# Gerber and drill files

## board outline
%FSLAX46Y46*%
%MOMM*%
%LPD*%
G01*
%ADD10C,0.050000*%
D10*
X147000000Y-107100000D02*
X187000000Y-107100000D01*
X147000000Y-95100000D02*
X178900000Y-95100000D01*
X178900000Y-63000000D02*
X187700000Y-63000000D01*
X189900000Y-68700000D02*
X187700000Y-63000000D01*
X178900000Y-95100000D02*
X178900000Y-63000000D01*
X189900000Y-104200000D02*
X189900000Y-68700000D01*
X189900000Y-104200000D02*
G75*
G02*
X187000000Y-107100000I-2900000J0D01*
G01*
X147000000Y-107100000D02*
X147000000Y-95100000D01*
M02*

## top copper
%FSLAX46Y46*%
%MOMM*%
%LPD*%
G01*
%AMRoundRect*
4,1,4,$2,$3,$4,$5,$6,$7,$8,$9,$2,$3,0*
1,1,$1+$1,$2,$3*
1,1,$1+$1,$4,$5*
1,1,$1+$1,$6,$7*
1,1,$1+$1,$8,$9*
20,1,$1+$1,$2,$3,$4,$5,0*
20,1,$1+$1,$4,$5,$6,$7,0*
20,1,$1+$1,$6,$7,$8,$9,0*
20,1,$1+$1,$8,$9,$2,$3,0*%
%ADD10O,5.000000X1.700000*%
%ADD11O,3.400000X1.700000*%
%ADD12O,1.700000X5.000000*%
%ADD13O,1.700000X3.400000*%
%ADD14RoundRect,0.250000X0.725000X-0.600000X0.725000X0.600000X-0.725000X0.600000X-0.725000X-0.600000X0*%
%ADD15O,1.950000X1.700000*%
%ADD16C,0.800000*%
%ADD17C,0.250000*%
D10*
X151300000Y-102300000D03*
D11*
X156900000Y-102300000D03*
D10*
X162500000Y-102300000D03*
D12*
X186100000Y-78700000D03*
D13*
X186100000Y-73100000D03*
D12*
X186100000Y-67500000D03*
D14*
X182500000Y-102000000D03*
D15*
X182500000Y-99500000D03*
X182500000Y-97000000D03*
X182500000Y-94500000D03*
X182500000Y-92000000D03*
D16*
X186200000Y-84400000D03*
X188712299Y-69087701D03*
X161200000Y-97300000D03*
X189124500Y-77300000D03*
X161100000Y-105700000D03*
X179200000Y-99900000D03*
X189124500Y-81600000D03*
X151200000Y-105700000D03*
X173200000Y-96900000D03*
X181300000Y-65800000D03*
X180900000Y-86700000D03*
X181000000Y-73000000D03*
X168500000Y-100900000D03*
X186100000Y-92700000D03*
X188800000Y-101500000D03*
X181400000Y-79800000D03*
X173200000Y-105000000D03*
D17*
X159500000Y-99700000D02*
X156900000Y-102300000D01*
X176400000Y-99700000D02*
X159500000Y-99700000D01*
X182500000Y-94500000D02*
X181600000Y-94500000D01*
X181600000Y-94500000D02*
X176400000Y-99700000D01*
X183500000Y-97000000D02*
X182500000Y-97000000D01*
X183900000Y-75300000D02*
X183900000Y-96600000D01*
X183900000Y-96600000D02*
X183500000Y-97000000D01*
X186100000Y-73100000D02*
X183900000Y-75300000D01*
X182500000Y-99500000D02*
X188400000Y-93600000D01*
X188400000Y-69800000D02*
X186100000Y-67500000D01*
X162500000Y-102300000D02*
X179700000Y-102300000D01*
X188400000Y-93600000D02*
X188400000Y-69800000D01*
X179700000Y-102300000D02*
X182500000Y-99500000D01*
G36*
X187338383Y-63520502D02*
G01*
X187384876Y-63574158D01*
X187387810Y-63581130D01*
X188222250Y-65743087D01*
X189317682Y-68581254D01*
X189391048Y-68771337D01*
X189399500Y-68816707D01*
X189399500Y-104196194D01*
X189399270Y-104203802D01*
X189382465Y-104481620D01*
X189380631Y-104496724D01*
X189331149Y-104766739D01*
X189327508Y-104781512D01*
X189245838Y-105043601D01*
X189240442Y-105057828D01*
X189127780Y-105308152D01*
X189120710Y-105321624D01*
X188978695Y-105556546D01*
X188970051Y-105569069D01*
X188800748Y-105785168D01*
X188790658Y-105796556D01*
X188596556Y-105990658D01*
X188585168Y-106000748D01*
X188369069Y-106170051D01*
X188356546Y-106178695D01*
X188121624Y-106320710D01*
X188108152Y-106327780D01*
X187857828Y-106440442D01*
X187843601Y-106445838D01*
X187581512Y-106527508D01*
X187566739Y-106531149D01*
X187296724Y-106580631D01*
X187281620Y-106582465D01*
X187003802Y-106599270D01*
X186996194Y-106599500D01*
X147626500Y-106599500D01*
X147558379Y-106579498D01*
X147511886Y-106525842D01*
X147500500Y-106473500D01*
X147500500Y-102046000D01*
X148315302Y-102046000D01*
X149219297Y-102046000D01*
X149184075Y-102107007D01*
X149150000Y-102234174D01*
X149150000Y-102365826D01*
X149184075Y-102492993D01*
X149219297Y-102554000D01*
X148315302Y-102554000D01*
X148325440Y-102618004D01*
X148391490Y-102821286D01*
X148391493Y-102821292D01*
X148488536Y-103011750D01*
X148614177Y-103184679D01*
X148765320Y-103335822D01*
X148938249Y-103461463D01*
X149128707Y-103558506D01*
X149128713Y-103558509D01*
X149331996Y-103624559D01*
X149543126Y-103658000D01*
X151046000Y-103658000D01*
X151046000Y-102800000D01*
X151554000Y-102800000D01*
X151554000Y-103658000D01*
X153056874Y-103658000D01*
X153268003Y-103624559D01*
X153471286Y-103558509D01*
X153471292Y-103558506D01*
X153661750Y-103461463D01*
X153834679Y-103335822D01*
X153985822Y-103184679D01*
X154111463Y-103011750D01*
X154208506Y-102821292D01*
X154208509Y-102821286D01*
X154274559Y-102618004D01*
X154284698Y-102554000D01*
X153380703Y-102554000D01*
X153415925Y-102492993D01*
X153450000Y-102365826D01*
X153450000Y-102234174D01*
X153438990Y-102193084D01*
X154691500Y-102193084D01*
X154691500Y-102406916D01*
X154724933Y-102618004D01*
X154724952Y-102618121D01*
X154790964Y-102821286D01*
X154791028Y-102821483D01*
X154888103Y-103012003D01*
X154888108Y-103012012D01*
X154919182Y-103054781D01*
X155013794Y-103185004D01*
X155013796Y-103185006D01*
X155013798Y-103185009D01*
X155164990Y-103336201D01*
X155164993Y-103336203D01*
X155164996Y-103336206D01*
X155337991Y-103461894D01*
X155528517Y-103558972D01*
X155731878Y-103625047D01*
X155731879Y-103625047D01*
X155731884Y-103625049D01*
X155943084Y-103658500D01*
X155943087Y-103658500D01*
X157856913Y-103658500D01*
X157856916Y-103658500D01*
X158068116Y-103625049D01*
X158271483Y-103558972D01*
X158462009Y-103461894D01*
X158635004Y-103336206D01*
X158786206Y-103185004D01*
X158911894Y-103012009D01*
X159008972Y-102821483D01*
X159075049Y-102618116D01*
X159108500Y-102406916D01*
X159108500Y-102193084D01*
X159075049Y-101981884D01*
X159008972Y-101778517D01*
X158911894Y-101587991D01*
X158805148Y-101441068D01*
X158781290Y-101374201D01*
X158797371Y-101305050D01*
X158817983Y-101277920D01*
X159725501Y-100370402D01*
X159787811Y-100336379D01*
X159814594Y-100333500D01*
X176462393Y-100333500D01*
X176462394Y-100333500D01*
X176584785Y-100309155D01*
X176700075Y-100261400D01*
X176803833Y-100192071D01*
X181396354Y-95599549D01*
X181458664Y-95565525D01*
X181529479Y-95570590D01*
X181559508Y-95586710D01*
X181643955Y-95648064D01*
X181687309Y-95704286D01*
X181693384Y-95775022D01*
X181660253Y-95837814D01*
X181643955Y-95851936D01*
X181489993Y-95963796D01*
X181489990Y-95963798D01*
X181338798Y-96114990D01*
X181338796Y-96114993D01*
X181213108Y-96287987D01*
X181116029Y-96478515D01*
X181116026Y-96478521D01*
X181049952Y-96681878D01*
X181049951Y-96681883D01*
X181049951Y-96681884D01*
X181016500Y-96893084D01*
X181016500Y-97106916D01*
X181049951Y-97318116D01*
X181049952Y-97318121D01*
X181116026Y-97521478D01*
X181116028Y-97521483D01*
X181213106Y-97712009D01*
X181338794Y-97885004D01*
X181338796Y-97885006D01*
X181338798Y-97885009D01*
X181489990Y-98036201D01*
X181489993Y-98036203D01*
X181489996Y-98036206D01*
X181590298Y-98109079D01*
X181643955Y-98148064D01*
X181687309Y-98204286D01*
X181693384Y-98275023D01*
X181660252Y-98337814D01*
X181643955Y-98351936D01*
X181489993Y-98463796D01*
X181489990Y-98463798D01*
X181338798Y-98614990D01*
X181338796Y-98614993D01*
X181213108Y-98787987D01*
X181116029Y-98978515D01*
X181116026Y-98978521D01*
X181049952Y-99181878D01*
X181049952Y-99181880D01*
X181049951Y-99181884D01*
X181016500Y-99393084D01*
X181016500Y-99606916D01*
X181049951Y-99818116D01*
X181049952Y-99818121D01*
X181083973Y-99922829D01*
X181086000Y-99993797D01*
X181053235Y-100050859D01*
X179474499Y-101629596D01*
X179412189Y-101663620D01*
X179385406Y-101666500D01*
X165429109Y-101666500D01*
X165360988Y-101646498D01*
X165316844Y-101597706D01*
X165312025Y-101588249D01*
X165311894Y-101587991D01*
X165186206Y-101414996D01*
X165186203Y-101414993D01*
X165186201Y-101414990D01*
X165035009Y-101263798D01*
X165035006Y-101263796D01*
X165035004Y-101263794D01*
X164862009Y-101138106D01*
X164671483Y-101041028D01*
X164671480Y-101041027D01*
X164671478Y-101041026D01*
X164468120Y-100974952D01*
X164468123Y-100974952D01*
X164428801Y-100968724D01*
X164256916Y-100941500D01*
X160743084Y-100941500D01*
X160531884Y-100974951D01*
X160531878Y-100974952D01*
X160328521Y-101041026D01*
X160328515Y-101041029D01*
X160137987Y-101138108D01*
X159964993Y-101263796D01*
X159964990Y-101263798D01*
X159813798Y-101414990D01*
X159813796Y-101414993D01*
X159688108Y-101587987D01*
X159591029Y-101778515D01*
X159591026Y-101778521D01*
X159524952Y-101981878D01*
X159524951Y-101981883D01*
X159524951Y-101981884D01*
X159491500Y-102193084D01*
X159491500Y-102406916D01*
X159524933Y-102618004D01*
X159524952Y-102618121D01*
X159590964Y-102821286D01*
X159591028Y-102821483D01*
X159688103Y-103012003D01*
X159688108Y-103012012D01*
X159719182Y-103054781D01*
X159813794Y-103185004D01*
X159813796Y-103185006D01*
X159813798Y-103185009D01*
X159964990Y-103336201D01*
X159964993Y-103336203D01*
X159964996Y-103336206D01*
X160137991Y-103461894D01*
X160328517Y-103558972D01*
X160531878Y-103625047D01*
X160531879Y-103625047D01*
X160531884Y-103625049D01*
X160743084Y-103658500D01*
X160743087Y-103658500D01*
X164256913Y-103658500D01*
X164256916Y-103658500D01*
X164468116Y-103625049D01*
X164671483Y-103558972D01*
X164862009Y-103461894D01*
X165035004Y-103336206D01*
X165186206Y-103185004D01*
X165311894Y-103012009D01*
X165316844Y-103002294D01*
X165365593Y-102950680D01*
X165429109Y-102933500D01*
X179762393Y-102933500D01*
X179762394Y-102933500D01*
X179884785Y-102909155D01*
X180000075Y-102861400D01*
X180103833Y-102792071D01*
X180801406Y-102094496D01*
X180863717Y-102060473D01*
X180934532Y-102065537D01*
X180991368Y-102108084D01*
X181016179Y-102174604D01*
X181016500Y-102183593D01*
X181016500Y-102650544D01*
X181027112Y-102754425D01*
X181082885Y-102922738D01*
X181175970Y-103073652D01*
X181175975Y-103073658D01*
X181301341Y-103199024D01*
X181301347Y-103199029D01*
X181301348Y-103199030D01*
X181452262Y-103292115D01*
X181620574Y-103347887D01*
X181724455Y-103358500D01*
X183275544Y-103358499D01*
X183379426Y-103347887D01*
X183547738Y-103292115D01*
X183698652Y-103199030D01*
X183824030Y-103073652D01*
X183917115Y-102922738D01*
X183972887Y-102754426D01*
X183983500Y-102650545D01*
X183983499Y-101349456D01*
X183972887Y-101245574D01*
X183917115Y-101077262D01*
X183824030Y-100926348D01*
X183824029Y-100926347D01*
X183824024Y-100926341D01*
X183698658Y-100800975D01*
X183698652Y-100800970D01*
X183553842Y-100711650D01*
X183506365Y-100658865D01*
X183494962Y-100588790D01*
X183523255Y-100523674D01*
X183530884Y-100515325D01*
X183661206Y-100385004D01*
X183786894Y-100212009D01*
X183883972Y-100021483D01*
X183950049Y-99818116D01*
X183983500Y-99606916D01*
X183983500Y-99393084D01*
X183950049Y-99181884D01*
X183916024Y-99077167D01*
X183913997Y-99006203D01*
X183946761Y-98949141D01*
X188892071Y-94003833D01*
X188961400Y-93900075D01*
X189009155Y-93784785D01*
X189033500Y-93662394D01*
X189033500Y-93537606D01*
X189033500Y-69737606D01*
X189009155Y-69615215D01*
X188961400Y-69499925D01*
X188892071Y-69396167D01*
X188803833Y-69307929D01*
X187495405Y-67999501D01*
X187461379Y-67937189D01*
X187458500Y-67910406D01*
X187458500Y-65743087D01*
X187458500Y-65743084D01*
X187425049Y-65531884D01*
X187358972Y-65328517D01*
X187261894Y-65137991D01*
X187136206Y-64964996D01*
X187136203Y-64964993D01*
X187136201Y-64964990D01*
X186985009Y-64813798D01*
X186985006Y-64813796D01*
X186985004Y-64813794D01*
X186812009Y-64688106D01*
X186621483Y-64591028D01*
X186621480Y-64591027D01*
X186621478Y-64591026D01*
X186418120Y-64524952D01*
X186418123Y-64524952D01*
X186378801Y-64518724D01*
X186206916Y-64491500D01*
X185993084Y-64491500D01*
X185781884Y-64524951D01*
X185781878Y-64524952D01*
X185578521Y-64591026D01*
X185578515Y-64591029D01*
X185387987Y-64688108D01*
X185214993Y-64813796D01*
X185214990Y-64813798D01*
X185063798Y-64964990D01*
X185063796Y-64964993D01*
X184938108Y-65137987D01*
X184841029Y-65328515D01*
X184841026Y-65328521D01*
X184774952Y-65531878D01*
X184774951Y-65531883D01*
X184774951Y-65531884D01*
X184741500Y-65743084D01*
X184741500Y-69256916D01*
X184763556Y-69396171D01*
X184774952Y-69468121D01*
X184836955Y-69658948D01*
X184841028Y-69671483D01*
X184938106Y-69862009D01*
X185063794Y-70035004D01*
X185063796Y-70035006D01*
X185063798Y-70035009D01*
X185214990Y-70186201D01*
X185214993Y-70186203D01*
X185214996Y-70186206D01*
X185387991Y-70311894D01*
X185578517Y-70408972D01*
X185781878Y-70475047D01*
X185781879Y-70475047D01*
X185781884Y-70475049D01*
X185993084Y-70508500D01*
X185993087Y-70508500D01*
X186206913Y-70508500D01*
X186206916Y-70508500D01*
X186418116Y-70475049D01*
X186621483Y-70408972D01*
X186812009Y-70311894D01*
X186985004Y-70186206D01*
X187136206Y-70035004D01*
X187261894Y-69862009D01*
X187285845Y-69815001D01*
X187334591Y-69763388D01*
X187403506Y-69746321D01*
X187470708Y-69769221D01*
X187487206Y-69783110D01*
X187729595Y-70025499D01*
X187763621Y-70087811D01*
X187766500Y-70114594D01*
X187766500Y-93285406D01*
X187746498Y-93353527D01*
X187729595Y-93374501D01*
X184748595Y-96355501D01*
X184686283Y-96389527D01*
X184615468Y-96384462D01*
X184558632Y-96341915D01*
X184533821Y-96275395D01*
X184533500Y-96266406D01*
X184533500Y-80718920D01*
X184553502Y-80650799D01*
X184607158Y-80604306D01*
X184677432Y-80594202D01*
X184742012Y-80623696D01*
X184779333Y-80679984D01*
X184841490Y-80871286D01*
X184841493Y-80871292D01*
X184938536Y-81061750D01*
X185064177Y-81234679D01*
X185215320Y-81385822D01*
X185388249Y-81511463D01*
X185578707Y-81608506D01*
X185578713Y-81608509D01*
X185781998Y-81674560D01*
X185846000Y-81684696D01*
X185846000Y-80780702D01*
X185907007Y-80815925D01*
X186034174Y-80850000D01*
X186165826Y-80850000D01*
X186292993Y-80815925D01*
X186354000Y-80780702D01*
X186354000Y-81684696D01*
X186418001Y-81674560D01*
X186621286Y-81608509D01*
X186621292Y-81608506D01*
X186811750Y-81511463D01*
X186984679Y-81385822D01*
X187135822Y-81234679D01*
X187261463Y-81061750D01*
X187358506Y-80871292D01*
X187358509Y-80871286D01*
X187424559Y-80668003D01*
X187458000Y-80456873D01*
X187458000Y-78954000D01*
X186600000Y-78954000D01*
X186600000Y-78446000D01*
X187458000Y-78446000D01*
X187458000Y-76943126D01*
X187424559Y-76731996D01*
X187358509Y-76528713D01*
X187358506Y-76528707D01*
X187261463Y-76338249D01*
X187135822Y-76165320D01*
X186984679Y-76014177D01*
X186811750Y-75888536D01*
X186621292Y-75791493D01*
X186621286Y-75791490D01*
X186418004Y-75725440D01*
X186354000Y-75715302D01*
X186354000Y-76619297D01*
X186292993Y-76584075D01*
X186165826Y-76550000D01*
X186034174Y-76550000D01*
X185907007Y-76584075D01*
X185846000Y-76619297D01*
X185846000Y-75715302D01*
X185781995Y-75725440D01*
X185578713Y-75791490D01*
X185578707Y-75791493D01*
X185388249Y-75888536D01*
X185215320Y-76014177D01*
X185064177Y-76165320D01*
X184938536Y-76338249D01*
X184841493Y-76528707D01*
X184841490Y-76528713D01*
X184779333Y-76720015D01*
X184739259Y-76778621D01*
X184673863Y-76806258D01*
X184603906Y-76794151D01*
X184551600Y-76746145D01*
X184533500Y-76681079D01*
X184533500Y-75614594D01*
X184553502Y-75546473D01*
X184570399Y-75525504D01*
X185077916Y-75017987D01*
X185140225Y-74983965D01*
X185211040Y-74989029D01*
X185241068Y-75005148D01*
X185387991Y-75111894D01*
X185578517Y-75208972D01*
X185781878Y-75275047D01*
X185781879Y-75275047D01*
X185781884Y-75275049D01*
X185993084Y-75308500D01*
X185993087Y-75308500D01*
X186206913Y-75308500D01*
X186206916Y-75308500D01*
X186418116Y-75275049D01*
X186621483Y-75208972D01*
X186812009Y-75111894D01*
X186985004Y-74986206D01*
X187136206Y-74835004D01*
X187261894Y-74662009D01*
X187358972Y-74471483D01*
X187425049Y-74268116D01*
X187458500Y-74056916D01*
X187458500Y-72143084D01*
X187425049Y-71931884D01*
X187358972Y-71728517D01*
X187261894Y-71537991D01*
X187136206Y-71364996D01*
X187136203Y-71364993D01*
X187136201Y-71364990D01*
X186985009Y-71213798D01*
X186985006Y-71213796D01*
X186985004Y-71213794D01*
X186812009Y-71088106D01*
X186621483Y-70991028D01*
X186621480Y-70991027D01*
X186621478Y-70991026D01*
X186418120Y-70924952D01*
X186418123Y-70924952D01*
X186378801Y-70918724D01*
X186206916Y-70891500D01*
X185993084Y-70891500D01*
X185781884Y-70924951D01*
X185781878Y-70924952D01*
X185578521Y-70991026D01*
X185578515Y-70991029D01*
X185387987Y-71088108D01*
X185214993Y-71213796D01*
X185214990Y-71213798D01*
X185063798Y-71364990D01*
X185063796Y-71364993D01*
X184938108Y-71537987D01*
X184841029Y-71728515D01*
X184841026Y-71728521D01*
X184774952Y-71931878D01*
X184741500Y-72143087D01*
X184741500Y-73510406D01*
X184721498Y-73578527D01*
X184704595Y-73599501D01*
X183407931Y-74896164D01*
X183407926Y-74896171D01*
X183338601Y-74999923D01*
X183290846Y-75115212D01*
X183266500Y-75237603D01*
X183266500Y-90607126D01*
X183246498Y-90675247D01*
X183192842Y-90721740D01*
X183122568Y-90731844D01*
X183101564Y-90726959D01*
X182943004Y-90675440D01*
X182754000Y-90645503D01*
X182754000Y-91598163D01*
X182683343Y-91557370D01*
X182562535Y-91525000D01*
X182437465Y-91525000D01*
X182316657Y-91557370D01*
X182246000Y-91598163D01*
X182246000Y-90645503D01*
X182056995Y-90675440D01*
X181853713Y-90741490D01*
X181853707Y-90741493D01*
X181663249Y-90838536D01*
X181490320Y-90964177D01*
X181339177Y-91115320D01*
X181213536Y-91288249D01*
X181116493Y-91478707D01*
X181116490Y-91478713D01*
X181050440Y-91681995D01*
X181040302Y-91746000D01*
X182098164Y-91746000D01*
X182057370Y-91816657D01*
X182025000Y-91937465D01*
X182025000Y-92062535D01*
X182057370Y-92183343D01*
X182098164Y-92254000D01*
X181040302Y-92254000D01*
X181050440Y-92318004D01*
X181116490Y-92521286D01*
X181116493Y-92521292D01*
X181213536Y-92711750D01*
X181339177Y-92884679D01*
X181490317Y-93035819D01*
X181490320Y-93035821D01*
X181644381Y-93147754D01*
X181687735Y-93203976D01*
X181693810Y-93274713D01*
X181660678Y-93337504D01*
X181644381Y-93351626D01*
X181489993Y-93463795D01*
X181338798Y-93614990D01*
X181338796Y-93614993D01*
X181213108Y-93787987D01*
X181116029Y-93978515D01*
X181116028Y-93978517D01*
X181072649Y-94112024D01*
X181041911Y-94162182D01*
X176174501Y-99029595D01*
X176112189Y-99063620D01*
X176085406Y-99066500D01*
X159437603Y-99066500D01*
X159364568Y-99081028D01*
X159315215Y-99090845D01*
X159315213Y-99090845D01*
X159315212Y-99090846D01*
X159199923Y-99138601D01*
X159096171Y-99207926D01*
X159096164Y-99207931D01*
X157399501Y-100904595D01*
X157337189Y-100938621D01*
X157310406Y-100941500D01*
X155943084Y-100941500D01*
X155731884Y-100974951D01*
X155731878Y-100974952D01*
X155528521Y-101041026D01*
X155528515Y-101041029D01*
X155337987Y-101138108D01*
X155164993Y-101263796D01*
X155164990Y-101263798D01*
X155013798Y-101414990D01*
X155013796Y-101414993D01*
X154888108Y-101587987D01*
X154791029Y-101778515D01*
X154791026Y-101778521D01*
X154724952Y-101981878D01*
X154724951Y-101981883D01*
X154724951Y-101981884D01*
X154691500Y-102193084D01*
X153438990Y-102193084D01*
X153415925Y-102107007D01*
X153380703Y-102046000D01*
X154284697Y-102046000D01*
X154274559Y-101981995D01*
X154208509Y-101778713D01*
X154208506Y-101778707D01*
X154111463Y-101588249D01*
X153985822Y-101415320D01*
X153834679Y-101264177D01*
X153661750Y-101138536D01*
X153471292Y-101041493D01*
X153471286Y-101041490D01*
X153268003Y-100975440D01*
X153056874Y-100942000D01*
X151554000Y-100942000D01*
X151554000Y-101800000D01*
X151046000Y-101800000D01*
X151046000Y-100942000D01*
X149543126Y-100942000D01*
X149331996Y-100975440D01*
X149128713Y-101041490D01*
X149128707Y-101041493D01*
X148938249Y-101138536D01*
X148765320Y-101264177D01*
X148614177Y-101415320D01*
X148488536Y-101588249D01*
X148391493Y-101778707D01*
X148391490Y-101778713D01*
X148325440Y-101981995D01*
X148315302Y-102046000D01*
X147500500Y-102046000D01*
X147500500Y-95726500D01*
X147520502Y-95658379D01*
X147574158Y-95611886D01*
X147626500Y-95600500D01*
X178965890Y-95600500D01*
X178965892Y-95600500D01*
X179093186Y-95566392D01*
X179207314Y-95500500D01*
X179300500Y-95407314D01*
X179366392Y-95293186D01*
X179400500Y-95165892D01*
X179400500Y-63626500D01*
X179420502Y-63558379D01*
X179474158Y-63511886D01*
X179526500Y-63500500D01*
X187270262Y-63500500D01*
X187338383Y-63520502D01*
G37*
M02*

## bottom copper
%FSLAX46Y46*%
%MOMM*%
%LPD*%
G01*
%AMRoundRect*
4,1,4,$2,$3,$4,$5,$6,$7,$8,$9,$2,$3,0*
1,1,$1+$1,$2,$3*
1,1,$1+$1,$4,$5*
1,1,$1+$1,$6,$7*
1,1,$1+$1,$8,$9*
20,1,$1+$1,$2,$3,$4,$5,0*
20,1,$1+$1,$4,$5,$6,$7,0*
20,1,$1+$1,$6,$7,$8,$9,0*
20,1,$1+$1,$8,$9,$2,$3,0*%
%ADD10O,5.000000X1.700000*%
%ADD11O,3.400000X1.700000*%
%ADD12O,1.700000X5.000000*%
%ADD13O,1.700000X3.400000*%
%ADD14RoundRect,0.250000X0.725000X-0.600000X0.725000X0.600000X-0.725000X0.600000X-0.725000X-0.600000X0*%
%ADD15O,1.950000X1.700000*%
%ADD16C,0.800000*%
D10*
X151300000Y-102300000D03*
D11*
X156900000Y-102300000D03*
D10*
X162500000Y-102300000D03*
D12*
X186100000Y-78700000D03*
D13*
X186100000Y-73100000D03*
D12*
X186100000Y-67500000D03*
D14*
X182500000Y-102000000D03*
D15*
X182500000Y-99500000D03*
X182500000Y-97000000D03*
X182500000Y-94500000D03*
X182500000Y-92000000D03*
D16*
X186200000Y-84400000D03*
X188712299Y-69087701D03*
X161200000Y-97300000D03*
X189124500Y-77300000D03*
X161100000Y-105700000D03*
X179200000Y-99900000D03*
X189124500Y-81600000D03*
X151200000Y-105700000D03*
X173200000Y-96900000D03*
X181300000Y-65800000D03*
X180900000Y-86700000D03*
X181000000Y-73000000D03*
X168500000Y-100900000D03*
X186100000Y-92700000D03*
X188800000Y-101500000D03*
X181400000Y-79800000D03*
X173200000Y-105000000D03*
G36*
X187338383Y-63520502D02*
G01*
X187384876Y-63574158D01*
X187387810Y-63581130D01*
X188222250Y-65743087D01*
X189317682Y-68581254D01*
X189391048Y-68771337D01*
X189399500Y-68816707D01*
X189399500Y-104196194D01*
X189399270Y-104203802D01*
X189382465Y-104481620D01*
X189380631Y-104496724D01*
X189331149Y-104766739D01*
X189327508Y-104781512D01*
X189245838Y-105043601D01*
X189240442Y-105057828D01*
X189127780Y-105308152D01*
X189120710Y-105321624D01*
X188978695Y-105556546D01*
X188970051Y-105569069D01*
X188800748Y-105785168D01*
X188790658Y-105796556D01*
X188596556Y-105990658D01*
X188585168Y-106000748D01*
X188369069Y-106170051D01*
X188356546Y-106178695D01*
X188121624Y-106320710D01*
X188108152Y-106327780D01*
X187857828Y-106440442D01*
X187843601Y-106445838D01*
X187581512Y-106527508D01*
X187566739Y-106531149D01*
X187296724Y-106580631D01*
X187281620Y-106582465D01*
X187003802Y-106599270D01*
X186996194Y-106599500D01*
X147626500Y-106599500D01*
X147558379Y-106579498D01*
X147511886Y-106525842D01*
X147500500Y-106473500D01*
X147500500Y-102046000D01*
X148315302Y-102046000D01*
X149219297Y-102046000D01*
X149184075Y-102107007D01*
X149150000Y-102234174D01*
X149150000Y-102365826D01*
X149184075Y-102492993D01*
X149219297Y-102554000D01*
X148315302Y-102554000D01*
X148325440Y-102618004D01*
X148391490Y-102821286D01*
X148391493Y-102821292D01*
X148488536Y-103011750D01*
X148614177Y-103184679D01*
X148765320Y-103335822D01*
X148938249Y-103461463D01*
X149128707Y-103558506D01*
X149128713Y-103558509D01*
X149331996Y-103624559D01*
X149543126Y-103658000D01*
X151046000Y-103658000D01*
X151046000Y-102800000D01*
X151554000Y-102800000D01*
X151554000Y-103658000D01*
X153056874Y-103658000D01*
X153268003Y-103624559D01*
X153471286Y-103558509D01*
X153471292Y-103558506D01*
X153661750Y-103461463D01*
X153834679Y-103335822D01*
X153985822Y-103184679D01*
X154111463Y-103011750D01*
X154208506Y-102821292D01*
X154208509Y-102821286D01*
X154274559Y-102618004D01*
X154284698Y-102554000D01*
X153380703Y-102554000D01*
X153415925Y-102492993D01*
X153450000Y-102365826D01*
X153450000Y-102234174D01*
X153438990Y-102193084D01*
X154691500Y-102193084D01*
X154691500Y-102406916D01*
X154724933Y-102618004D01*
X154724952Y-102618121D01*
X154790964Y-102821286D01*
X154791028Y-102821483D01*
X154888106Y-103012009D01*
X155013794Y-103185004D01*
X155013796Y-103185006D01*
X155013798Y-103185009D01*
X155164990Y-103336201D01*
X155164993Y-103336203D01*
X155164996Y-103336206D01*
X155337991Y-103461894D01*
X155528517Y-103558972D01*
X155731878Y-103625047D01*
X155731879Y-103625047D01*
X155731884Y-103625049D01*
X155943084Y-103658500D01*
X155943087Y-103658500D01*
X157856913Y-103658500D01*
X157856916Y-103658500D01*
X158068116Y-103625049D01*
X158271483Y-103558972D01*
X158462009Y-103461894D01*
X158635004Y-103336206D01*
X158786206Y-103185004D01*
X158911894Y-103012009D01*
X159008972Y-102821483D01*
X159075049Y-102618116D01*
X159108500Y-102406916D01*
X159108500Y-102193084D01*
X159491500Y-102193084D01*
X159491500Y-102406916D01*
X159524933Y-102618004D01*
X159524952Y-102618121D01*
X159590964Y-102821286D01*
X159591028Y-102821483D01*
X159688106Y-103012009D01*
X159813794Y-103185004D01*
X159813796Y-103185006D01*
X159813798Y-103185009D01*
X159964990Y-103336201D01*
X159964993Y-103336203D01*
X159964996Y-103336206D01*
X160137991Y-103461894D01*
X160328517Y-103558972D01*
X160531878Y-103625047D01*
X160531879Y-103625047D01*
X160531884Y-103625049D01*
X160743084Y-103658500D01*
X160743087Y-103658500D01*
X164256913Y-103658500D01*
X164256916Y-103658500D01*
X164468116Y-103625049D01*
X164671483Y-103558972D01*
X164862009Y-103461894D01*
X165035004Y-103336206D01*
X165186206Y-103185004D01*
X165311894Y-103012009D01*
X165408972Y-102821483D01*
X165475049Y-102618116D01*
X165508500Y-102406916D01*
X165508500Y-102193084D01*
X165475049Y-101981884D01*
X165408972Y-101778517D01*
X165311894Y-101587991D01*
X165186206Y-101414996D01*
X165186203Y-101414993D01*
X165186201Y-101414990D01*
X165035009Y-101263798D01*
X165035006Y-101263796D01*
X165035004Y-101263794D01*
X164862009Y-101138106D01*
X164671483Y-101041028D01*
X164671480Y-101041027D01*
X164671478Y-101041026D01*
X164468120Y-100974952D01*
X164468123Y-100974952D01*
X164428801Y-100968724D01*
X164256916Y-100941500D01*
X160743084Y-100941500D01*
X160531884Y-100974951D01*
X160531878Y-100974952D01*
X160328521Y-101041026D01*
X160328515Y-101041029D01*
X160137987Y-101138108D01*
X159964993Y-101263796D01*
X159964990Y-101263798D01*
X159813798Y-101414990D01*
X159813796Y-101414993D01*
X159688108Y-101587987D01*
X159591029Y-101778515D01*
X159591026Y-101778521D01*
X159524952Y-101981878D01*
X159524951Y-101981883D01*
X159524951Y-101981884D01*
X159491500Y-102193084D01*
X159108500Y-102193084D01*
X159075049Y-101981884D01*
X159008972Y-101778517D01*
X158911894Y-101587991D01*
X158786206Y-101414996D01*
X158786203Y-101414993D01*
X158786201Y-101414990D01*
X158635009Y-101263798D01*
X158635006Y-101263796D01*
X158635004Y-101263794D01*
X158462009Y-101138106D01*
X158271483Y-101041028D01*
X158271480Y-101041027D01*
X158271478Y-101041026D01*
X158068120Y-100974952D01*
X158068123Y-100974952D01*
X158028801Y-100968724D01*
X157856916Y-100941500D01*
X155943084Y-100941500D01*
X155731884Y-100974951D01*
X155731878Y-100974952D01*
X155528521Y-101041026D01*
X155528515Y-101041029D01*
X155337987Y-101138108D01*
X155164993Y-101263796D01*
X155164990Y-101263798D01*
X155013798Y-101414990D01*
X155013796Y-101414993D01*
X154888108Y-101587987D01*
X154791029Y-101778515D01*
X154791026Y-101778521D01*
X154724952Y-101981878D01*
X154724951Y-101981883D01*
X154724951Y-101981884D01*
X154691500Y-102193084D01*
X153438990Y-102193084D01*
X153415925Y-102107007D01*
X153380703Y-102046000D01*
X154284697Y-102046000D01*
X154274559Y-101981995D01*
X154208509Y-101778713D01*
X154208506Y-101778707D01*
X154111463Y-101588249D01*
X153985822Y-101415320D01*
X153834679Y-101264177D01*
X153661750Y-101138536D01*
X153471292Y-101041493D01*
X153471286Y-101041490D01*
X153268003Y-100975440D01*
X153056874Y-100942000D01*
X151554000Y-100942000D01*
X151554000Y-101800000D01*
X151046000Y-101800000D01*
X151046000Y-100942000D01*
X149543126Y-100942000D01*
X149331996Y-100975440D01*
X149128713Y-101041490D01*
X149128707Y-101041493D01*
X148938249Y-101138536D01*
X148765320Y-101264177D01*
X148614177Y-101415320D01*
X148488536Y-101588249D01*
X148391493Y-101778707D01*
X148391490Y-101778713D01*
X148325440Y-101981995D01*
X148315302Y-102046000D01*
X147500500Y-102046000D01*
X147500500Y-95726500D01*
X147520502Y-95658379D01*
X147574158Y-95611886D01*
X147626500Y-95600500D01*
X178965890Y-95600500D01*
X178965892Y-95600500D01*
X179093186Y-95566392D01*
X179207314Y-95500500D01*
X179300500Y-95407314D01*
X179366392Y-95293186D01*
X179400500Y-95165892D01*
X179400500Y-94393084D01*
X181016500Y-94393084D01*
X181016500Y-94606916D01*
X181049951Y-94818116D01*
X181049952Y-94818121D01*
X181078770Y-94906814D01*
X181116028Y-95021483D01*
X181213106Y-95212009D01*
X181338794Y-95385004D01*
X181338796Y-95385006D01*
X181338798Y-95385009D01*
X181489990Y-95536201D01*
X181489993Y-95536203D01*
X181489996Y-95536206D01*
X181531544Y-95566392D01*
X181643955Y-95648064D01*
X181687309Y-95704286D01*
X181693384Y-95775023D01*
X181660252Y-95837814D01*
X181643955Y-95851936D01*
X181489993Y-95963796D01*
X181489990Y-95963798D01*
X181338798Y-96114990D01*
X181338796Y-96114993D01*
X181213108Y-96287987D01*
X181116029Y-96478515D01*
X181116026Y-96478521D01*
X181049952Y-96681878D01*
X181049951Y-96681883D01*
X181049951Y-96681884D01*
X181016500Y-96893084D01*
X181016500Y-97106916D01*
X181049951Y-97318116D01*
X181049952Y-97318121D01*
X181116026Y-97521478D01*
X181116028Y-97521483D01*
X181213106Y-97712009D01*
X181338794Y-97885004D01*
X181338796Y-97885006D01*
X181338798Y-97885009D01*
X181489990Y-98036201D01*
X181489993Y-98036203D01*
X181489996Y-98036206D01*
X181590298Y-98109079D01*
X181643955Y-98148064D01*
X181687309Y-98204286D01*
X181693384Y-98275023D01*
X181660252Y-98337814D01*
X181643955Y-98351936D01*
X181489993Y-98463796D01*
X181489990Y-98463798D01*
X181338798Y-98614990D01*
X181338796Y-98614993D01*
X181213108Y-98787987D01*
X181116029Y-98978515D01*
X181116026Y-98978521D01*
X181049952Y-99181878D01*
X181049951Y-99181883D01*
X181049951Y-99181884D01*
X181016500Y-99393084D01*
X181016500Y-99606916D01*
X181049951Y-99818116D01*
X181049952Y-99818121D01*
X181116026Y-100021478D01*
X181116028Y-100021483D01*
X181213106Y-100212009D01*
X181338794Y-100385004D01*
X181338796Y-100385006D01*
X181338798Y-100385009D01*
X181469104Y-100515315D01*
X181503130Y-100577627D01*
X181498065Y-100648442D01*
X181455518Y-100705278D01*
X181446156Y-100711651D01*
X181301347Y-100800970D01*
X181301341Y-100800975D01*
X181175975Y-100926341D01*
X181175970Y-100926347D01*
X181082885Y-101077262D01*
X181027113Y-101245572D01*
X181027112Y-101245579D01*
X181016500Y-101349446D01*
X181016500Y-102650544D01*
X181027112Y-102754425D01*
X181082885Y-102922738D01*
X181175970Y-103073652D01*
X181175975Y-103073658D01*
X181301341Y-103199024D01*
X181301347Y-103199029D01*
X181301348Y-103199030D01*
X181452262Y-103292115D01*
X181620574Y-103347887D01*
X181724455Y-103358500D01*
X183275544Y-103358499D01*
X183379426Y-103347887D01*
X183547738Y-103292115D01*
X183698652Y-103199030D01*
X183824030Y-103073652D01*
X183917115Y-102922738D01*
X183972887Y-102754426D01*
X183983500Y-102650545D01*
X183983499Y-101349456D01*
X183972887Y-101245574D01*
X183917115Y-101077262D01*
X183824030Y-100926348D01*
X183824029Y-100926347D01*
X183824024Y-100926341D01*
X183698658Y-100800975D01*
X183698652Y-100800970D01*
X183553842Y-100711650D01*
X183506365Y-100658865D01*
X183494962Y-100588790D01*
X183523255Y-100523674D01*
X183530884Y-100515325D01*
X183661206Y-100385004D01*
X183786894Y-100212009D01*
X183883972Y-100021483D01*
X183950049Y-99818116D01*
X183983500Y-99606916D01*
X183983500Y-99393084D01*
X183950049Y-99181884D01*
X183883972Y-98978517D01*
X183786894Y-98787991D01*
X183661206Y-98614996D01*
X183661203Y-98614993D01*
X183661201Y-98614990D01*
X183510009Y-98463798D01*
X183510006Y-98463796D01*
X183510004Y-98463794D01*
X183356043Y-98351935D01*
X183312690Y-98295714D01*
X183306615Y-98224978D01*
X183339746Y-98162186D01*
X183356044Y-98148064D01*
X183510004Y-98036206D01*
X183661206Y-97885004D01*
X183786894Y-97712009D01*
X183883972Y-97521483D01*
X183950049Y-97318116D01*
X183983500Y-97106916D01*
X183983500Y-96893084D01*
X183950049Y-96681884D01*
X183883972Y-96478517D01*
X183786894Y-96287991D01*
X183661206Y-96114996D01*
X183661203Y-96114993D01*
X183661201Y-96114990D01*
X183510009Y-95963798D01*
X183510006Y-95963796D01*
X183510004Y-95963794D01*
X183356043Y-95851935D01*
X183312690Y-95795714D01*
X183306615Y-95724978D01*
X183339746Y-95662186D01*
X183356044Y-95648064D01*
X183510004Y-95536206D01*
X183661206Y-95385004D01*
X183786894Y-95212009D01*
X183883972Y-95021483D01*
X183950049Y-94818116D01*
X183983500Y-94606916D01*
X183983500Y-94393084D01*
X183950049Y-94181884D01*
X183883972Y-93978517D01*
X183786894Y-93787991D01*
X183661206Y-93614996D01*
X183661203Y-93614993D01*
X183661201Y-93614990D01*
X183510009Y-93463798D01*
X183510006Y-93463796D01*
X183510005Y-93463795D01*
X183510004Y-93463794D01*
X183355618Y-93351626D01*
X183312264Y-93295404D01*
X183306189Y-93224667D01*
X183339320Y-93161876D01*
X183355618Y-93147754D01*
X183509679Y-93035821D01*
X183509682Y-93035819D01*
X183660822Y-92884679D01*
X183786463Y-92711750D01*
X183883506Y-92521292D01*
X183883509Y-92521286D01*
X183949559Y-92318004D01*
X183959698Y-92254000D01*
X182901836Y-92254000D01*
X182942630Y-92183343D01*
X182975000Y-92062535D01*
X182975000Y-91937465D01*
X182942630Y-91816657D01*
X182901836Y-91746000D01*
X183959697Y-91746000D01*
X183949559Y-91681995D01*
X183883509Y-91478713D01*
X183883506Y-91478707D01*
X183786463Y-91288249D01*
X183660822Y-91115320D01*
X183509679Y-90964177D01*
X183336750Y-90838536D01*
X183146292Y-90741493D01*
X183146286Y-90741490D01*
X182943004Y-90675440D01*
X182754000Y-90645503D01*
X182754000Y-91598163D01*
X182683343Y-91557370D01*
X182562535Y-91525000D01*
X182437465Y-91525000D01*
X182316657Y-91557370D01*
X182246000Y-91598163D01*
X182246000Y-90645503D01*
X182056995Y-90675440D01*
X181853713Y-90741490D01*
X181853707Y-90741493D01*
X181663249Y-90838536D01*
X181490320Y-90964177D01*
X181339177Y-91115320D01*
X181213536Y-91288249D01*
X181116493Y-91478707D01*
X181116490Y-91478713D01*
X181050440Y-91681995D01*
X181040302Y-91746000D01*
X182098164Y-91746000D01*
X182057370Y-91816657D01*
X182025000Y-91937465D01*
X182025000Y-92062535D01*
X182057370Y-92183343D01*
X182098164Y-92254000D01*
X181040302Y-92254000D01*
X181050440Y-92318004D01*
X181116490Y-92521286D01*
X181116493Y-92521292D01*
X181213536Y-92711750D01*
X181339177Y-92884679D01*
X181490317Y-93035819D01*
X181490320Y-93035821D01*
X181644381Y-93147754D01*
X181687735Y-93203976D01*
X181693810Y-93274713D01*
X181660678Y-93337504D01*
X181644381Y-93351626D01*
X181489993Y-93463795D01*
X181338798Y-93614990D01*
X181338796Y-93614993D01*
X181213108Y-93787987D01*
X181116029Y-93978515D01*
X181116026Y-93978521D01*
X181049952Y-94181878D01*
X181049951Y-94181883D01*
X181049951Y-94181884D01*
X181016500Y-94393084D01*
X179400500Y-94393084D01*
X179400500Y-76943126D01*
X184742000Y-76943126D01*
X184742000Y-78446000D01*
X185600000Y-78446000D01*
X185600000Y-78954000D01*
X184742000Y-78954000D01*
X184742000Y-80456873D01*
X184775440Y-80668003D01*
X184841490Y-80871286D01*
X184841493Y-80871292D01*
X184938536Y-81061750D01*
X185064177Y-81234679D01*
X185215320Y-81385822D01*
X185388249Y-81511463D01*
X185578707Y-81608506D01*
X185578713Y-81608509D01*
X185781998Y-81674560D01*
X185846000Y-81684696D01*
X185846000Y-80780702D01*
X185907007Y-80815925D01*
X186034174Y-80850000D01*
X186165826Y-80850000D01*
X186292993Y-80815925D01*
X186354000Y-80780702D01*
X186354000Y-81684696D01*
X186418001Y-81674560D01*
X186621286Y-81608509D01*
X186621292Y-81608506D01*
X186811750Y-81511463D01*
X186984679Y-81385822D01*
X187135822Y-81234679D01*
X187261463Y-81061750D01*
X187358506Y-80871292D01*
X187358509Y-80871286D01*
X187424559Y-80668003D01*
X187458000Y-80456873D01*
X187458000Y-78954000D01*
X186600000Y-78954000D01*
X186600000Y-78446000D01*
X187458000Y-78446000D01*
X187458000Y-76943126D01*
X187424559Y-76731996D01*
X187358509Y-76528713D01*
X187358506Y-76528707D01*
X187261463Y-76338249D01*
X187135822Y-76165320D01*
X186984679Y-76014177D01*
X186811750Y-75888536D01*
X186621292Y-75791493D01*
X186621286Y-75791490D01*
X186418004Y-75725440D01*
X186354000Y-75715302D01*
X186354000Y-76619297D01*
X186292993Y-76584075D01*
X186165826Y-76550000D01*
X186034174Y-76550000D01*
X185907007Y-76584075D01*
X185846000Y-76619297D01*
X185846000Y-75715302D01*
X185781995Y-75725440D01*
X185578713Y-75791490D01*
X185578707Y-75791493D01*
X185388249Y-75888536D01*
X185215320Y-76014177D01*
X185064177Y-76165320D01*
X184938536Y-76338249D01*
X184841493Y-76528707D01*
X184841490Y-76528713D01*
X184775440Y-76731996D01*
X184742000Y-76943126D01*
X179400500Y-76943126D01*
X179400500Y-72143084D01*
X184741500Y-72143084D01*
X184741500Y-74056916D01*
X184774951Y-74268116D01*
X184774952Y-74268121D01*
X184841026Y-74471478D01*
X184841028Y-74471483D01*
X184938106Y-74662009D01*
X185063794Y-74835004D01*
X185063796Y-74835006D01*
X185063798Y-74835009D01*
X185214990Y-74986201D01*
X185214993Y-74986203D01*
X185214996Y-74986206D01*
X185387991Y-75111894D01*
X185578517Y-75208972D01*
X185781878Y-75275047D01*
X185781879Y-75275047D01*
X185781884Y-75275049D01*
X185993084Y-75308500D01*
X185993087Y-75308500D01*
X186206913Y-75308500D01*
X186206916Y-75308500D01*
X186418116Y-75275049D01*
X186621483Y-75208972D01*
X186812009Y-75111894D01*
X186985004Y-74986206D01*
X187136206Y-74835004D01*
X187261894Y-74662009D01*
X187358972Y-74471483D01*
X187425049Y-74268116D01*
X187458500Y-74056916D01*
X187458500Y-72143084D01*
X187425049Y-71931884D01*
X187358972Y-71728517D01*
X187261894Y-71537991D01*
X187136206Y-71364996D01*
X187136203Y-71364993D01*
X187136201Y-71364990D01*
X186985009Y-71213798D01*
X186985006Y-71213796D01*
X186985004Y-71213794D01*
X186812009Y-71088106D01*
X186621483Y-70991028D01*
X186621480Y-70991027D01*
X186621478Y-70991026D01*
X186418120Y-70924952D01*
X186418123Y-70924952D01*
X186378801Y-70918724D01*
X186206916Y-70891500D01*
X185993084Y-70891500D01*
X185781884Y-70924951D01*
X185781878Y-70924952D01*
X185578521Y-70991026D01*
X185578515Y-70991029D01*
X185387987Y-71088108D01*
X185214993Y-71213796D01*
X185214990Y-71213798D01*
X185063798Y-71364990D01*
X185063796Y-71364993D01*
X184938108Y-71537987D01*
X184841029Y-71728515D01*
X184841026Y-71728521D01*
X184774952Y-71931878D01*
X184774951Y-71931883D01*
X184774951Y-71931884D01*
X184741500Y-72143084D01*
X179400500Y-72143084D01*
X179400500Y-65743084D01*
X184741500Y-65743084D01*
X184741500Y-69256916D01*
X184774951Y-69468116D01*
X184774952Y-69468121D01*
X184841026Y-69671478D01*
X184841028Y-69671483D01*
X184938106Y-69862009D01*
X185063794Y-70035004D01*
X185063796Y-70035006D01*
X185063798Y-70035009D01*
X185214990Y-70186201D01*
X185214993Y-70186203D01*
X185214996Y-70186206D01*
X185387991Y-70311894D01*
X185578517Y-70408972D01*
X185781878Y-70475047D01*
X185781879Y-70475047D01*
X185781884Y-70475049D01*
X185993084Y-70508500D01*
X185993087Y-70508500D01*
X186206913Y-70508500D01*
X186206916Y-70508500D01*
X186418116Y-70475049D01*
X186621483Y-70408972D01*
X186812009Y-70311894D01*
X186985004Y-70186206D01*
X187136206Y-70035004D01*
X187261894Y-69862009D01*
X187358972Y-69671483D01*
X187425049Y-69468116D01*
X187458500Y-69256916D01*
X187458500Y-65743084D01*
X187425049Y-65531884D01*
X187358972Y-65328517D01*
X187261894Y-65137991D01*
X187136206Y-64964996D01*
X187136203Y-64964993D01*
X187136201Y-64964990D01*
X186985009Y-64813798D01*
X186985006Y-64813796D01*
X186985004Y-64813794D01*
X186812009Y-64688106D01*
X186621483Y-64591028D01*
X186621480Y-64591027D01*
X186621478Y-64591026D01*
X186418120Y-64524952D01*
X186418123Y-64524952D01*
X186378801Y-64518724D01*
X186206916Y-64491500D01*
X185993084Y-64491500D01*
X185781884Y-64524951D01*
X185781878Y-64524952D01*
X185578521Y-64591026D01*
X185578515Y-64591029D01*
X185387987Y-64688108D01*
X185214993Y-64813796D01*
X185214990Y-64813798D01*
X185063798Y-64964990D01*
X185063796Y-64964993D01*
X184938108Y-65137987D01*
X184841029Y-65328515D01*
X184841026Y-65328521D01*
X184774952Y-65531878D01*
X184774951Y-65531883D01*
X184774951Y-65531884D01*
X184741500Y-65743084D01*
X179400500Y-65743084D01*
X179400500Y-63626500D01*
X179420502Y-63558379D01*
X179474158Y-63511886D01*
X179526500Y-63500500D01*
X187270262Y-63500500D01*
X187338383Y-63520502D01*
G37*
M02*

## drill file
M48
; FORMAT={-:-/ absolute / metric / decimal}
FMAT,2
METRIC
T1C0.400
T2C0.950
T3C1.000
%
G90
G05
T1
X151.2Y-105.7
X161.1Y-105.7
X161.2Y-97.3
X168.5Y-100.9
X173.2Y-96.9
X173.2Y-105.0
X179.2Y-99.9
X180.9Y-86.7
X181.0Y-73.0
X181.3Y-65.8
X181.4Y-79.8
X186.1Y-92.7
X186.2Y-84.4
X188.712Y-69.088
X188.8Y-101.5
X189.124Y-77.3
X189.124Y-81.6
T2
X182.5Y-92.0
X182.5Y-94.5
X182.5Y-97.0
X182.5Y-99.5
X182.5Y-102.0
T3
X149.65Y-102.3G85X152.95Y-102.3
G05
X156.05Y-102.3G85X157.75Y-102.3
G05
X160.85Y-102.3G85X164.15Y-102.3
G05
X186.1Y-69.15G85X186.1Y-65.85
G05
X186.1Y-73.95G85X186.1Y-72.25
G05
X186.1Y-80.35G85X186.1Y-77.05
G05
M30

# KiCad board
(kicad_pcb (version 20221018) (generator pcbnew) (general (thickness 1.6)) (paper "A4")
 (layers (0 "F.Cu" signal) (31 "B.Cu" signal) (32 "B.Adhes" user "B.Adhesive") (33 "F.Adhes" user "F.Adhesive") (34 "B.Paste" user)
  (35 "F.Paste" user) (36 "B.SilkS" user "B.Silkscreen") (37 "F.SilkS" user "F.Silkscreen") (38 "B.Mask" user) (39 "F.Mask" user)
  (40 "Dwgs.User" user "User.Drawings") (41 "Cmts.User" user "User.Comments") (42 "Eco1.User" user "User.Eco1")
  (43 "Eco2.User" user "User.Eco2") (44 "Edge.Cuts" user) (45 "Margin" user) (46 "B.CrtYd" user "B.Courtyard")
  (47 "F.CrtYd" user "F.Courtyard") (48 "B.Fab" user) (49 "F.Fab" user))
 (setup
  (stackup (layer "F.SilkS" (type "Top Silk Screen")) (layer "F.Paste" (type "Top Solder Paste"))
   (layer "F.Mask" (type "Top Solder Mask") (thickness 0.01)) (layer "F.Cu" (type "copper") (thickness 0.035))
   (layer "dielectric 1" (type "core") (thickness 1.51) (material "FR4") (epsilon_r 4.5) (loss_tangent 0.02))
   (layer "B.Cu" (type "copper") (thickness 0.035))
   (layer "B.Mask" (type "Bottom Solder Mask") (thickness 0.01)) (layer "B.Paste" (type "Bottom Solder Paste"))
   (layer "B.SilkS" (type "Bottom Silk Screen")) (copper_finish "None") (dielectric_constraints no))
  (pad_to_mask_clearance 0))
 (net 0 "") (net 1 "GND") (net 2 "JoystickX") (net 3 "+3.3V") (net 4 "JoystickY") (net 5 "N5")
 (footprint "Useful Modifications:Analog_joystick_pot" (layer "F.Cu") (at 156.9 102.3 90)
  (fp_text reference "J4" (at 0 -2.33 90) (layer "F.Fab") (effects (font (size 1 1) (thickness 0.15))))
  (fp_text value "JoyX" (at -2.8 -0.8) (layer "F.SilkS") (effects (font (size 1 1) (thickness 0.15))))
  (pad "1" thru_hole oval (at 0 -5.6 90) (size 1.7 5) (drill oval 1 4.3) (layers "*.Cu" "*.Mask") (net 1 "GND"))
  (pad "2" thru_hole oval (at 0 0 90) (size 1.7 3.4) (drill oval 1 2.7) (layers "*.Cu" "*.Mask") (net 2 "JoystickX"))
  (pad "3" thru_hole oval (at 0 5.6 90) (size 1.7 5) (drill oval 1 4.3) (layers "*.Cu" "*.Mask") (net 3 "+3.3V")))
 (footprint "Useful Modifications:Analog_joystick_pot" (layer "F.Cu") (at 186.1 73.1 180)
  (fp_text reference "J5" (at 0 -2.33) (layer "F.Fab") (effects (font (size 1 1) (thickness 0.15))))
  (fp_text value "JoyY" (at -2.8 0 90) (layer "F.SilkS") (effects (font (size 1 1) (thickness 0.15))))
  (pad "1" thru_hole oval (at 0 -5.6 180) (size 1.7 5) (drill oval 1 4.3) (layers "*.Cu" "*.Mask") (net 1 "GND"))
  (pad "2" thru_hole oval (at 0 0 180) (size 1.7 3.4) (drill oval 1 2.7) (layers "*.Cu" "*.Mask") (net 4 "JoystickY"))
  (pad "3" thru_hole oval (at 0 5.6 180) (size 1.7 5) (drill oval 1 4.3) (layers "*.Cu" "*.Mask") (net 3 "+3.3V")))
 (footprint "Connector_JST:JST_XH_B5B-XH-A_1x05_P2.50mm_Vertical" (layer "F.Cu") (at 182.5 102 90)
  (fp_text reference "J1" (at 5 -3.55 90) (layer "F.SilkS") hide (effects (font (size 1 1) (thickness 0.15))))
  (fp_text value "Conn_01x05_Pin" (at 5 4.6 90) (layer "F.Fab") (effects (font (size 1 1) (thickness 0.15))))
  (pad "1" thru_hole roundrect (at 0 0 90) (size 1.7 1.95) (drill 0.95) (layers "*.Cu" "*.Mask") (roundrect_rratio 0.147059) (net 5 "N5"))
  (pad "2" thru_hole oval (at 2.5 0 90) (size 1.7 1.95) (drill 0.95) (layers "*.Cu" "*.Mask") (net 3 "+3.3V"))
  (pad "3" thru_hole oval (at 5 0 90) (size 1.7 1.95) (drill 0.95) (layers "*.Cu" "*.Mask") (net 4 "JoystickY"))
  (pad "4" thru_hole oval (at 7.5 0 90) (size 1.7 1.95) (drill 0.95) (layers "*.Cu" "*.Mask") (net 2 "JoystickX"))
  (pad "5" thru_hole oval (at 10 0 90) (size 1.7 1.95) (drill 0.95) (layers "*.Cu" "*.Mask") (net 1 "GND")))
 (gr_line (start 147 107.1) (end 187 107.1) (stroke (width 0.05) (type default)) (layer "Edge.Cuts"))
 (gr_line (start 147 95.1) (end 178.9 95.1) (stroke (width 0.05) (type default)) (layer "Edge.Cuts"))
 (gr_line (start 178.9 63) (end 187.7 63) (stroke (width 0.05) (type default)) (layer "Edge.Cuts"))
 (gr_line (start 189.9 68.7) (end 187.7 63) (stroke (width 0.05) (type default)) (layer "Edge.Cuts"))
 (gr_line (start 178.9 95.1) (end 178.9 63) (stroke (width 0.05) (type default)) (layer "Edge.Cuts"))
 (gr_line (start 189.9 104.2) (end 189.9 68.7) (stroke (width 0.05) (type default)) (layer "Edge.Cuts"))
 (gr_arc (start 189.9 104.2) (mid 189.05061 106.25061) (end 187 107.1) (stroke (width 0.05) (type default)) (layer "Edge.Cuts"))
 (gr_line (start 147 107.1) (end 147 95.1) (stroke (width 0.05) (type default)) (layer "Edge.Cuts"))
 (via (at 186.2 84.4) (size 0.8) (drill 0.4) (layers "F.Cu" "B.Cu") (free) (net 1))
 (via (at 188.712299 69.087701) (size 0.8) (drill 0.4) (layers "F.Cu" "B.Cu") (free) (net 1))
 (via (at 161.2 97.3) (size 0.8) (drill 0.4) (layers "F.Cu" "B.Cu") (free) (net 1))
 (via (at 189.1245 77.3) (size 0.8) (drill 0.4) (layers "F.Cu" "B.Cu") (free) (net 1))
 (via (at 161.1 105.7) (size 0.8) (drill 0.4) (layers "F.Cu" "B.Cu") (free) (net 1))
 (via (at 179.2 99.9) (size 0.8) (drill 0.4) (layers "F.Cu" "B.Cu") (free) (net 1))
 (via (at 189.1245 81.6) (size 0.8) (drill 0.4) (layers "F.Cu" "B.Cu") (free) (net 1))
 (via (at 151.2 105.7) (size 0.8) (drill 0.4) (layers "F.Cu" "B.Cu") (free) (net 1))
 (via (at 173.2 96.9) (size 0.8) (drill 0.4) (layers "F.Cu" "B.Cu") (free) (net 1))
 (via (at 181.3 65.8) (size 0.8) (drill 0.4) (layers "F.Cu" "B.Cu") (free) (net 1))
 (via (at 180.9 86.7) (size 0.8) (drill 0.4) (layers "F.Cu" "B.Cu") (free) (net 1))
 (via (at 181 73) (size 0.8) (drill 0.4) (layers "F.Cu" "B.Cu") (free) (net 1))
 (via (at 168.5 100.9) (size 0.8) (drill 0.4) (layers "F.Cu" "B.Cu") (free) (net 1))
 (via (at 186.1 92.7) (size 0.8) (drill 0.4) (layers "F.Cu" "B.Cu") (free) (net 1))
 (via (at 188.8 101.5) (size 0.8) (drill 0.4) (layers "F.Cu" "B.Cu") (free) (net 1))
 (via (at 181.4 79.8) (size 0.8) (drill 0.4) (layers "F.Cu" "B.Cu") (free) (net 1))
 (via (at 173.2 105) (size 0.8) (drill 0.4) (layers "F.Cu" "B.Cu") (free) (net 1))
 (segment (start 159.5 99.7) (end 156.9 102.3) (width 0.25) (layer "F.Cu") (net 2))
 (segment (start 176.4 99.7) (end 159.5 99.7) (width 0.25) (layer "F.Cu") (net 2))
 (segment (start 182.5 94.5) (end 181.6 94.5) (width 0.25) (layer "F.Cu") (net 2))
 (segment (start 181.6 94.5) (end 176.4 99.7) (width 0.25) (layer "F.Cu") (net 2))
 (segment (start 183.5 97) (end 182.5 97) (width 0.25) (layer "F.Cu") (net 4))
 (segment (start 183.9 75.3) (end 183.9 96.6) (width 0.25) (layer "F.Cu") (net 4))
 (segment (start 183.9 96.6) (end 183.5 97) (width 0.25) (layer "F.Cu") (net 4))
 (segment (start 186.1 73.1) (end 183.9 75.3) (width 0.25) (layer "F.Cu") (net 4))
 (segment (start 182.5 99.5) (end 188.4 93.6) (width 0.25) (layer "F.Cu") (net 3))
 (segment (start 188.4 69.8) (end 186.1 67.5) (width 0.25) (layer "F.Cu") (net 3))
 (segment (start 162.5 102.3) (end 179.7 102.3) (width 0.25) (layer "F.Cu") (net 3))
 (segment (start 188.4 93.6) (end 188.4 69.8) (width 0.25) (layer "F.Cu") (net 3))
 (segment (start 179.7 102.3) (end 182.5 99.5) (width 0.25) (layer "F.Cu") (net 3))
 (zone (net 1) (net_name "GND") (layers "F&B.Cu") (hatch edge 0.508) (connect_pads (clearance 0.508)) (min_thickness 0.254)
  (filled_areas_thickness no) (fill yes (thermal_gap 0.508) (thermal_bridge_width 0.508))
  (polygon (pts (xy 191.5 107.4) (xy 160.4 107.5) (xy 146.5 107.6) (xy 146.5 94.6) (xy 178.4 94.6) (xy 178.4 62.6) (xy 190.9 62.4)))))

